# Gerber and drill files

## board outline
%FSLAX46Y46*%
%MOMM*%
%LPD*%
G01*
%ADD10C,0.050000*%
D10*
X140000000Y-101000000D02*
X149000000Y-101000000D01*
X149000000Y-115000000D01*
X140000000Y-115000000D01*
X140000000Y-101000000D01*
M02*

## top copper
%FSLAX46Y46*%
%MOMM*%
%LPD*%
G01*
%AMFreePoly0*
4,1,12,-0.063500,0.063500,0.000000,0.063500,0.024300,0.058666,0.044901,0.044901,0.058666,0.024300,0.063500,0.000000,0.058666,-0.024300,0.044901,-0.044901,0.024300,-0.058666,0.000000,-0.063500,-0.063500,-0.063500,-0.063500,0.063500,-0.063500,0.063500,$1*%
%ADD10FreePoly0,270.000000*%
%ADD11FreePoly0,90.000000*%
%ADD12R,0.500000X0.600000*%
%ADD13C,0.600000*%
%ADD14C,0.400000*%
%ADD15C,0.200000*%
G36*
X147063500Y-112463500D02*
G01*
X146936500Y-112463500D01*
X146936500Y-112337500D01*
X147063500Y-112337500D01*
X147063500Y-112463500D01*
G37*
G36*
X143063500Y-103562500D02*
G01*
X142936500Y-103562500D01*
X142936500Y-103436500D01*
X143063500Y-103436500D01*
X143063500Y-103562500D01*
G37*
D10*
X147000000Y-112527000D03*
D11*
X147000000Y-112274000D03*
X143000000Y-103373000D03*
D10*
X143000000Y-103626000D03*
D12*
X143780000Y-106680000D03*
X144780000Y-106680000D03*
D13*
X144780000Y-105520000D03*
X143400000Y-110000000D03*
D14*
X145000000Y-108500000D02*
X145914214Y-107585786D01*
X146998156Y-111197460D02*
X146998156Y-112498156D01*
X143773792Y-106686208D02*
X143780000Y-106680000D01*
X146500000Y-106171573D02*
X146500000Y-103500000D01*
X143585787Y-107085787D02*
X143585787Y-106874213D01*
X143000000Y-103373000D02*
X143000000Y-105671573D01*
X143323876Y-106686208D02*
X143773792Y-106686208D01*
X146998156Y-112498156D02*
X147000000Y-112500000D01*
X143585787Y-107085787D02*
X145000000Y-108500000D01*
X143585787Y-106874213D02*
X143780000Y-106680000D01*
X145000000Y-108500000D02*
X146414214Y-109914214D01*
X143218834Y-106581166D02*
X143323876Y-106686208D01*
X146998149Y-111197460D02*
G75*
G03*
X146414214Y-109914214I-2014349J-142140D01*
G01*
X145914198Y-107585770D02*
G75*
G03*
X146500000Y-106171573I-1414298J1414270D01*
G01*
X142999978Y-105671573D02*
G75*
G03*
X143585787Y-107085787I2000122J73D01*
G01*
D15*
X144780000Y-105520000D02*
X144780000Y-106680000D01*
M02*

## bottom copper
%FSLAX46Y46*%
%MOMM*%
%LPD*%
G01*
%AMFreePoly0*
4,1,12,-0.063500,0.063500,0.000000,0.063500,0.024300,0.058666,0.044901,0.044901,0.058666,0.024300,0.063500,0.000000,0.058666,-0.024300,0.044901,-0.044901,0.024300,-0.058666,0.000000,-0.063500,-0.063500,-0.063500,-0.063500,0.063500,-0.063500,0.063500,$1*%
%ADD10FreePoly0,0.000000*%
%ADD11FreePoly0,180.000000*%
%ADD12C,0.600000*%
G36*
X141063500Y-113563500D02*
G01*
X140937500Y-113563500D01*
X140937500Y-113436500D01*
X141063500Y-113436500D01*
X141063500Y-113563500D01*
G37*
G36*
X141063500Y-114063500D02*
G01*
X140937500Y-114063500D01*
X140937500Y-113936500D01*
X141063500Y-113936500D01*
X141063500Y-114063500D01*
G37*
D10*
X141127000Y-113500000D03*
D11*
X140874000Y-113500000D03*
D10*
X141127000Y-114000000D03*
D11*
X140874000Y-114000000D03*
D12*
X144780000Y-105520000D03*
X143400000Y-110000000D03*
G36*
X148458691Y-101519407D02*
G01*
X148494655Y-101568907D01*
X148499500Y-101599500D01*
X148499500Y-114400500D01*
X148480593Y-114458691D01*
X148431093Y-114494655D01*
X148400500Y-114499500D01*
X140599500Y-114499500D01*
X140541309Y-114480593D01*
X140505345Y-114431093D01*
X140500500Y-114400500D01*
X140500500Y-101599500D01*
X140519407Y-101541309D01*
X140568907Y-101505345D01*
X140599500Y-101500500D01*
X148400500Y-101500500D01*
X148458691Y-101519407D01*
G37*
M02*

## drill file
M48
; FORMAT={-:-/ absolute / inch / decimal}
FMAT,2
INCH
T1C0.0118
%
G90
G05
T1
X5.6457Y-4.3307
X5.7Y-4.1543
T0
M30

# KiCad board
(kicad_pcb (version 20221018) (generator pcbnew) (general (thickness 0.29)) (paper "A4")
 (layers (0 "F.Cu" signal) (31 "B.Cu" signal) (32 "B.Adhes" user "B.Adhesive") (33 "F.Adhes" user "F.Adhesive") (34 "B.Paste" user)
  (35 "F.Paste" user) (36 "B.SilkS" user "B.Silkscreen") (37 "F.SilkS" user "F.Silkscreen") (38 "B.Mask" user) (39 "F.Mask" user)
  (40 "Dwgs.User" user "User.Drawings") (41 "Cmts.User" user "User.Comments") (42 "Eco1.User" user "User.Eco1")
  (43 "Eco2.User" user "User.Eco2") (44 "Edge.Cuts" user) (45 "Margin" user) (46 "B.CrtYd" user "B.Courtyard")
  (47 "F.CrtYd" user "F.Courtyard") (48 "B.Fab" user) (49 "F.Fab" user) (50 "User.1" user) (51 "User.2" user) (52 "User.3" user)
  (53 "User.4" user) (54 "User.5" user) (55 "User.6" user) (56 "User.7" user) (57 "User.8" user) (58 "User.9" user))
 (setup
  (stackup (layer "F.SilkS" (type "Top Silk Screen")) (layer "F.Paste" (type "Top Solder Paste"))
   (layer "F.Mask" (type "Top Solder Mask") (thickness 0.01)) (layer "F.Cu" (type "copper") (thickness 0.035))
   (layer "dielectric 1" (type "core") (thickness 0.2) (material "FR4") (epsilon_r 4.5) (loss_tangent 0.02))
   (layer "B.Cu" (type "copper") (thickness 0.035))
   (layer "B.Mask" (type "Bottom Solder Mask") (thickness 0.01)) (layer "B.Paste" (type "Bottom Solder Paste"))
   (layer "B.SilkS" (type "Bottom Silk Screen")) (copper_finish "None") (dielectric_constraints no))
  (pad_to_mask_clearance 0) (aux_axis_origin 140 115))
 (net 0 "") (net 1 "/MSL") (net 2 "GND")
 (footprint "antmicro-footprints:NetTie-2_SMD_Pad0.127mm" (layer "F.Cu") (at 147 112.4 90) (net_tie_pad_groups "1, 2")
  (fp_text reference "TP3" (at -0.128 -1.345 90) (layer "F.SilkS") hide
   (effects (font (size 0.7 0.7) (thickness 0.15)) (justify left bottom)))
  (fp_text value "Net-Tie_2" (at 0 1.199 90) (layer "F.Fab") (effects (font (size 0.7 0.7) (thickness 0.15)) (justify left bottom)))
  (fp_poly
   (pts (xy -0.0635 -0.0635) (xy 0.0625 -0.0635) (xy 0.0625 0.0635) (xy -0.0635 0.0635)) (stroke (width 0) (type solid)) (fill solid)
   (layer "F.Cu"))
  (pad "1" smd roundrect (at -0.127 0 270) (size 0.127 0.127) (layers "F.Cu") (roundrect_rratio 0.5) (chamfer_ratio 0)
   (chamfer top_left bottom_left) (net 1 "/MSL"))
  (pad "2" smd roundrect (at 0.126 0 90) (size 0.127 0.127) (layers "F.Cu") (roundrect_rratio 0.5) (chamfer_ratio 0)
   (chamfer top_left bottom_left) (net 1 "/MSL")))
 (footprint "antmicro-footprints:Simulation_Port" (layer "F.Cu") (at 146.5 103.25 180)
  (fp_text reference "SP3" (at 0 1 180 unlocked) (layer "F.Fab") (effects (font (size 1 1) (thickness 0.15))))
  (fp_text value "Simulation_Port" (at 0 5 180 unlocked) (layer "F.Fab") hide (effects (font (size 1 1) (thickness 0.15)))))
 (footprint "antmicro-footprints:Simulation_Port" (layer "F.Cu") (at 147 112.75)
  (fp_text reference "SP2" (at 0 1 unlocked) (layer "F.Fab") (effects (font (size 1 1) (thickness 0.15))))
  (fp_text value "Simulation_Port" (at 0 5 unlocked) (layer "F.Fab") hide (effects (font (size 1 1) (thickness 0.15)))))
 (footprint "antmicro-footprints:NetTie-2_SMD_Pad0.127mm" (layer "F.Cu") (at 143 103.5 -90) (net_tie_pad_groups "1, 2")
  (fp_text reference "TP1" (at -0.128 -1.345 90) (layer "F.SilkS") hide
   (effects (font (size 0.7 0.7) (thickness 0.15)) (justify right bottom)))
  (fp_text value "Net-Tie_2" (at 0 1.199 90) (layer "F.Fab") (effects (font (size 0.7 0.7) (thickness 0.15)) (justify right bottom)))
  (fp_poly
   (pts (xy -0.0635 -0.0635) (xy 0.0625 -0.0635) (xy 0.0625 0.0635) (xy -0.0635 0.0635)) (stroke (width 0) (type solid)) (fill solid)
   (layer "F.Cu"))
  (pad "1" smd roundrect (at -0.127 0 90) (size 0.127 0.127) (layers "F.Cu") (roundrect_rratio 0.5) (chamfer_ratio 0)
   (chamfer top_left bottom_left) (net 1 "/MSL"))
  (pad "2" smd roundrect (at 0.126 0 270) (size 0.127 0.127) (layers "F.Cu") (roundrect_rratio 0.5) (chamfer_ratio 0)
   (chamfer top_left bottom_left) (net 1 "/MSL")))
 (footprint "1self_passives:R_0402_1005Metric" (layer "F.Cu") (at 144.28 106.68)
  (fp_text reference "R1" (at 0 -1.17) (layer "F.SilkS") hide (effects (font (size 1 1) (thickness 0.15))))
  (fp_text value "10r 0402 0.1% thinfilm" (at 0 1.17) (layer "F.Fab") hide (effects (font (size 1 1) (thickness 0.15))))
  (pad "1" smd rect (at -0.5 0) (size 0.5 0.6) (layers "F.Cu" "F.Paste" "F.Mask") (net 1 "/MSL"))
  (pad "2" smd rect (at 0.5 0) (size 0.5 0.6) (layers "F.Cu" "F.Paste" "F.Mask") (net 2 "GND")))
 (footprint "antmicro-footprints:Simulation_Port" (layer "F.Cu") (at 143 103.25 180)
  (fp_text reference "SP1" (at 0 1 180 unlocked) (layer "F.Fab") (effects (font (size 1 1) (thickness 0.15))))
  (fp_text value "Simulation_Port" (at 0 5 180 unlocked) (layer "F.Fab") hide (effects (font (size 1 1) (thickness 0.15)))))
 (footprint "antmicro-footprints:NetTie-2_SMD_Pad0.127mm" (layer "B.Cu") (at 141 113.5 180) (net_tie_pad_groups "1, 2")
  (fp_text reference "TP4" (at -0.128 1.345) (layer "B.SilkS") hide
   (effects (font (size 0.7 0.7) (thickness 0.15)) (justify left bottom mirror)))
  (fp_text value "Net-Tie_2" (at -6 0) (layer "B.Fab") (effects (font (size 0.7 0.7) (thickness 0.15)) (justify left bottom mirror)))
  (fp_poly
   (pts (xy -0.0635 0.0635) (xy 0.0625 0.0635) (xy 0.0625 -0.0635) (xy -0.0635 -0.0635)) (stroke (width 0) (type solid)) (fill solid)
   (layer "B.Cu"))
  (pad "1" smd roundrect (at -0.127 0) (size 0.127 0.127) (layers "B.Cu") (roundrect_rratio 0.5) (chamfer_ratio 0)
   (chamfer top_left bottom_left) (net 2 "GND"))
  (pad "2" smd roundrect (at 0.126 0 180) (size 0.127 0.127) (layers "B.Cu") (roundrect_rratio 0.5) (chamfer_ratio 0)
   (chamfer top_left bottom_left) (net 2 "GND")))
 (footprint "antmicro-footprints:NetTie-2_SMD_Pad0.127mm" (layer "B.Cu") (at 141 114 180) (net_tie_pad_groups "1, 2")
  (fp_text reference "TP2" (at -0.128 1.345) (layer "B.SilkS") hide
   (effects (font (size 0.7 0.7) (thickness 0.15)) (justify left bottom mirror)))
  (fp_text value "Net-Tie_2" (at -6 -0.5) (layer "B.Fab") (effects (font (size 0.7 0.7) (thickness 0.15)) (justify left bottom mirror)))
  (fp_poly
   (pts (xy -0.0635 0.0635) (xy 0.0625 0.0635) (xy 0.0625 -0.0635) (xy -0.0635 -0.0635)) (stroke (width 0) (type solid)) (fill solid)
   (layer "B.Cu"))
  (pad "1" smd roundrect (at -0.127 0) (size 0.127 0.127) (layers "B.Cu") (roundrect_rratio 0.5) (chamfer_ratio 0)
   (chamfer top_left bottom_left) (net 2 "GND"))
  (pad "2" smd roundrect (at 0.126 0 180) (size 0.127 0.127) (layers "B.Cu") (roundrect_rratio 0.5) (chamfer_ratio 0)
   (chamfer top_left bottom_left) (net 2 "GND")))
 (gr_rect (start 140 101) (end 149 115) (stroke (width 0.05) (type solid)) (fill none) (layer "Edge.Cuts"))
 (segment (start 145 108.5) (end 145.914214 107.585786) (width 0.4) (layer "F.Cu") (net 1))
 (segment (start 146.998156 111.19746) (end 146.998156 112.498156) (width 0.4) (layer "F.Cu") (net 1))
 (segment (start 143.773792 106.686208) (end 143.78 106.68) (width 0.4) (layer "F.Cu") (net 1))
 (segment (start 146.5 106.171573) (end 146.5 103.5) (width 0.4) (layer "F.Cu") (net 1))
 (segment (start 143.585787 107.085787) (end 143.585787 106.874213) (width 0.4) (layer "F.Cu") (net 1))
 (segment (start 143 103.373) (end 143 105.671573) (width 0.4) (layer "F.Cu") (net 1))
 (segment (start 143.323876 106.686208) (end 143.773792 106.686208) (width 0.4) (layer "F.Cu") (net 1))
 (segment (start 146.998156 112.498156) (end 147 112.5) (width 0.4) (layer "F.Cu") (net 1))
 (segment (start 143.585787 107.085787) (end 145 108.5) (width 0.4) (layer "F.Cu") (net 1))
 (segment (start 143.585787 106.874213) (end 143.78 106.68) (width 0.4) (layer "F.Cu") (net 1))
 (segment (start 145 108.5) (end 146.414214 109.914214) (width 0.4) (layer "F.Cu") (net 1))
 (segment (start 143.218834 106.581166) (end 143.323876 106.686208) (width 0.4) (layer "F.Cu") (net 1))
 (arc (start 146.414214 109.914214) (mid 146.82172 110.503015) (end 146.998156 111.19746) (width 0.4) (layer "F.Cu") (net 1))
 (arc (start 145.914214 107.585786) (mid 146.34775 106.936938) (end 146.5 106.171573) (width 0.4) (layer "F.Cu") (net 1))
 (arc (start 143 105.671573) (mid 143.15225 106.436939) (end 143.585787 107.085787) (width 0.4) (layer "F.Cu") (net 1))
 (segment (start 144.78 105.52) (end 144.78 106.68) (width 0.2) (layer "F.Cu") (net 2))
 (via (at 144.78 105.52) (size 0.6) (drill 0.3) (layers "F.Cu" "B.Cu") (free) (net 2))
 (via (at 143.4 110) (size 0.6) (drill 0.3) (layers "F.Cu" "B.Cu") (free) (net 2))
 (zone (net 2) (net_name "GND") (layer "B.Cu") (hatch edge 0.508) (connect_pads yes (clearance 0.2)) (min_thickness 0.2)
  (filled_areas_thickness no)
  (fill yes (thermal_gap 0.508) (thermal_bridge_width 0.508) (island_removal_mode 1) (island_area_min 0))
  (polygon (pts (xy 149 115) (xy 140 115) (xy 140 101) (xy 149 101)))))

